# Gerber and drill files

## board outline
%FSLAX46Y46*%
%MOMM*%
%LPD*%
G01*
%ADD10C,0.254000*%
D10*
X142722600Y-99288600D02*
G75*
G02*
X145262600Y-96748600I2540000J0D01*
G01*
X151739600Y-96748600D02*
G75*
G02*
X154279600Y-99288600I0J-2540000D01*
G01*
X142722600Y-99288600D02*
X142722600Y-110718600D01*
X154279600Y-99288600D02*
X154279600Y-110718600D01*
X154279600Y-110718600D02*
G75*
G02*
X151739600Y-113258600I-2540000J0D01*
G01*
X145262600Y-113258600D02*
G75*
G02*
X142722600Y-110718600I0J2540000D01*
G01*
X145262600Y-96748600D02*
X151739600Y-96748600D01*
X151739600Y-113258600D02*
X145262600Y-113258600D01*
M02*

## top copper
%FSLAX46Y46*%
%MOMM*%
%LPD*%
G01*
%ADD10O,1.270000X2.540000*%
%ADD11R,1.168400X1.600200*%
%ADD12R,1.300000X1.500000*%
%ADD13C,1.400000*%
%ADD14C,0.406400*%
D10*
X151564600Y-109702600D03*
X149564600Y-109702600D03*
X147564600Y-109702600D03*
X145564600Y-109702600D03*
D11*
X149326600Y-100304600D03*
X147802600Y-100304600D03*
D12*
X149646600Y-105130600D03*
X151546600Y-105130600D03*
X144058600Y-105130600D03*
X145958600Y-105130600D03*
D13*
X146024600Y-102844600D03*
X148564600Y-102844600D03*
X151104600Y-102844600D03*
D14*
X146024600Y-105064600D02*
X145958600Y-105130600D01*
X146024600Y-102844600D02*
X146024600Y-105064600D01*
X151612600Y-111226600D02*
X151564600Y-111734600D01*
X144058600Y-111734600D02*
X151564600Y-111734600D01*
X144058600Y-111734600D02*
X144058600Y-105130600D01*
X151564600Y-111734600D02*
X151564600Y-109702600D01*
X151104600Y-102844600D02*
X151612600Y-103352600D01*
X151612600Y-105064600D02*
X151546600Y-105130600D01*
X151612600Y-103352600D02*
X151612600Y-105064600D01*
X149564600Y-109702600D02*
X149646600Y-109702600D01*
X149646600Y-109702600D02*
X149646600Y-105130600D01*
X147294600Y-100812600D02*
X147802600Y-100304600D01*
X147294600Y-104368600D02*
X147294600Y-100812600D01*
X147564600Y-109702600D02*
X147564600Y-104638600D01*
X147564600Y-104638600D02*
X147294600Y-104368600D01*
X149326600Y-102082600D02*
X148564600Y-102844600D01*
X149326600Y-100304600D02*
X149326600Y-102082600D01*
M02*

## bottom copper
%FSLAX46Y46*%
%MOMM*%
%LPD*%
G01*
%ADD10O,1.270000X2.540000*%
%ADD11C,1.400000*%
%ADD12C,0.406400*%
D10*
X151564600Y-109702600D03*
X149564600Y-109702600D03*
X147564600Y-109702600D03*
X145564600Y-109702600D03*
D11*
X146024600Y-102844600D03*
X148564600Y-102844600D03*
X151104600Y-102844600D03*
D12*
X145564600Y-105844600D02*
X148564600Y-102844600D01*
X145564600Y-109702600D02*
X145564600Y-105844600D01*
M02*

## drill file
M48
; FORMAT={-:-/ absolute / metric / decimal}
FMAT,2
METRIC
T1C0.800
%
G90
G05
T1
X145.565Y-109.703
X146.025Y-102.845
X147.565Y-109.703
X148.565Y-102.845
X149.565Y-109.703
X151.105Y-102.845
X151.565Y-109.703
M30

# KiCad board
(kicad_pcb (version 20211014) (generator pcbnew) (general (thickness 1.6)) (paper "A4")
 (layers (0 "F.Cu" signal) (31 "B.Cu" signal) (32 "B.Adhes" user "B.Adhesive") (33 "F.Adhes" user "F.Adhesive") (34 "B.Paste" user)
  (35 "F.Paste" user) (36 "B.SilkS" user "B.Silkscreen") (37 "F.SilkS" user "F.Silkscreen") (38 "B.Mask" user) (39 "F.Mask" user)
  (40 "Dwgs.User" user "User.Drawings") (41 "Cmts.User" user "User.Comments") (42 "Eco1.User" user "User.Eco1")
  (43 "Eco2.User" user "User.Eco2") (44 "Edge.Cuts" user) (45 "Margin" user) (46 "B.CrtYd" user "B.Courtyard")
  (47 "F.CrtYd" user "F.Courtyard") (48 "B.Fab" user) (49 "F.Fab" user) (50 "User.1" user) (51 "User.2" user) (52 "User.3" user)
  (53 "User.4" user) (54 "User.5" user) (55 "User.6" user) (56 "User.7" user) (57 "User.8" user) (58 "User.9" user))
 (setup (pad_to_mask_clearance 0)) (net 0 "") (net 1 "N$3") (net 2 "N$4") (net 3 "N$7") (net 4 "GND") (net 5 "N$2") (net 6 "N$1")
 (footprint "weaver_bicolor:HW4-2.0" (layer "F.Cu") (at 148.5646 109.7026 180)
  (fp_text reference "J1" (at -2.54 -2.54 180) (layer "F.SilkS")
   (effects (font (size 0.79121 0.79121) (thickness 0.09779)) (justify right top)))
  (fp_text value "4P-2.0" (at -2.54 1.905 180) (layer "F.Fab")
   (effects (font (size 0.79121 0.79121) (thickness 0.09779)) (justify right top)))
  (pad "1" thru_hole oval (at -3 0 270) (size 2.54 1.27) (drill 0.8) (layers *.Cu *.Mask) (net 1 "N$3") (solder_mask_margin 0.1016))
  (pad "2" thru_hole oval (at -1 0 270) (size 2.54 1.27) (drill 0.8) (layers *.Cu *.Mask) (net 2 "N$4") (solder_mask_margin 0.1016))
  (pad "3" thru_hole oval (at 1 0 270) (size 2.54 1.27) (drill 0.8) (layers *.Cu *.Mask) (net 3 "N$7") (solder_mask_margin 0.1016))
  (pad "4" thru_hole oval (at 3 0 270) (size 2.54 1.27) (drill 0.8) (layers *.Cu *.Mask) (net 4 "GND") (solder_mask_margin 0.1016)))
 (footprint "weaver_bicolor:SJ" (layer "F.Cu") (at 148.5646 100.3046 180)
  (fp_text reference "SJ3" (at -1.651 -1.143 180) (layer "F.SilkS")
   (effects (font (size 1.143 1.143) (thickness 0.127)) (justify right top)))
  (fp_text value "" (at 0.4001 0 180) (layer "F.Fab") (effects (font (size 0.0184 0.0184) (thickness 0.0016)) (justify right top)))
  (pad "1" smd rect (at -0.762 0 180) (size 1.1684 1.6002) (layers "F.Cu" "F.Paste" "F.Mask") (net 4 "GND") (solder_mask_margin 0.1016))
  (pad "2" smd rect (at 0.762 0 180) (size 1.1684 1.6002) (layers "F.Cu" "F.Paste" "F.Mask") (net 3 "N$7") (solder_mask_margin 0.1016)))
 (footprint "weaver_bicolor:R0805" (layer "F.Cu") (at 150.5966 105.1306)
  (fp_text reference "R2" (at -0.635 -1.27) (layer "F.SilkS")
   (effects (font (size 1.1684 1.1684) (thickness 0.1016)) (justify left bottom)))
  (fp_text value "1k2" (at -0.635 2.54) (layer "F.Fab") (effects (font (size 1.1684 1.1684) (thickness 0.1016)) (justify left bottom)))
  (pad "1" smd rect (at -0.95 0) (size 1.3 1.5) (layers "F.Cu" "F.Paste" "F.Mask") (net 2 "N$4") (solder_mask_margin 0.1016))
  (pad "2" smd rect (at 0.95 0) (size 1.3 1.5) (layers "F.Cu" "F.Paste" "F.Mask") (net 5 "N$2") (solder_mask_margin 0.1016)))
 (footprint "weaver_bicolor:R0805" (layer "F.Cu") (at 145.0086 105.1306)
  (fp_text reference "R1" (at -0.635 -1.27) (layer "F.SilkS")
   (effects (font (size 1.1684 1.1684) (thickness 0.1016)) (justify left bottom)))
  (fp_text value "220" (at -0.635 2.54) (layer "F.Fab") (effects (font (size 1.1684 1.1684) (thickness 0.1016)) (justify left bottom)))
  (pad "1" smd rect (at -0.95 0) (size 1.3 1.5) (layers "F.Cu" "F.Paste" "F.Mask") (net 1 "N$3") (solder_mask_margin 0.1016))
  (pad "2" smd rect (at 0.95 0) (size 1.3 1.5) (layers "F.Cu" "F.Paste" "F.Mask") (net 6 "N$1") (solder_mask_margin 0.1016)))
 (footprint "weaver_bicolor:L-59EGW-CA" (layer "B.Cu") (at 148.5646 102.8446 -90)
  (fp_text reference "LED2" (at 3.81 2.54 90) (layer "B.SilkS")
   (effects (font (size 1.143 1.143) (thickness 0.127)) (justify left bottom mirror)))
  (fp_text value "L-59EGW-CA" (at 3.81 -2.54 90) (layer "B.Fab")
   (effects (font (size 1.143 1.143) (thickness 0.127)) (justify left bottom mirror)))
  (pad "1" thru_hole circle (at 0 2.54 180) (size 1.4 1.4) (drill 0.8) (layers *.Cu *.Mask) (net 6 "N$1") (solder_mask_margin 0.1016))
  (pad "2" thru_hole circle (at 0 0 180) (size 1.4 1.4) (drill 0.8) (layers *.Cu *.Mask) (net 4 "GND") (solder_mask_margin 0.1016))
  (pad "3" thru_hole circle (at 0 -2.54 180) (size 1.4 1.4) (drill 0.8) (layers *.Cu *.Mask) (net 5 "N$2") (solder_mask_margin 0.1016)))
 (gr_arc (start 142.7226 99.2886) (mid 143.466549 97.492549) (end 145.2626 96.7486) (layer "Edge.Cuts") (width 0.254))
 (gr_arc (start 151.7396 96.7486) (mid 153.535651 97.492549) (end 154.2796 99.2886) (layer "Edge.Cuts") (width 0.254))
 (gr_line (start 142.7226 99.2886) (end 142.7226 110.7186) (layer "Edge.Cuts") (width 0.254))
 (gr_line (start 154.2796 99.2886) (end 154.2796 110.7186) (layer "Edge.Cuts") (width 0.254))
 (gr_arc (start 154.2796 110.7186) (mid 153.535651 112.514651) (end 151.7396 113.2586) (layer "Edge.Cuts") (width 0.254))
 (gr_arc (start 145.2626 113.2586) (mid 143.466549 112.514651) (end 142.7226 110.7186) (layer "Edge.Cuts") (width 0.254))
 (gr_line (start 145.2626 96.7486) (end 151.7396 96.7486) (layer "Edge.Cuts") (width 0.254))
 (gr_line (start 151.7396 113.2586) (end 145.2626 113.2586) (layer "Edge.Cuts") (width 0.254))
 (segment (start 146.0246 105.0646) (end 145.9586 105.1306) (width 0.4064) (layer "F.Cu") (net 6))
 (segment (start 146.0246 102.8446) (end 146.0246 105.0646) (width 0.4064) (layer "F.Cu") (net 6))
 (segment (start 151.6126 111.2266) (end 151.5646 111.7346) (width 0.4064) (layer "F.Cu") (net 1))
 (segment (start 144.0586 111.7346) (end 151.5646 111.7346) (width 0.4064) (layer "F.Cu") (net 1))
 (segment (start 144.0586 111.7346) (end 144.0586 105.1306) (width 0.4064) (layer "F.Cu") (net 1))
 (segment (start 151.5646 111.7346) (end 151.5646 109.7026) (width 0.4064) (layer "F.Cu") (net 1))
 (segment (start 151.1046 102.8446) (end 151.6126 103.3526) (width 0.4064) (layer "F.Cu") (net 5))
 (segment (start 151.6126 105.0646) (end 151.5466 105.1306) (width 0.4064) (layer "F.Cu") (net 5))
 (segment (start 151.6126 103.3526) (end 151.6126 105.0646) (width 0.4064) (layer "F.Cu") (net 5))
 (segment (start 149.5646 109.7026) (end 149.6466 109.7026) (width 0.4064) (layer "F.Cu") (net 2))
 (segment (start 149.6466 109.7026) (end 149.6466 105.1306) (width 0.4064) (layer "F.Cu") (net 2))
 (segment (start 147.2946 100.8126) (end 147.8026 100.3046) (width 0.4064) (layer "F.Cu") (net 3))
 (segment (start 147.2946 104.3686) (end 147.2946 100.8126) (width 0.4064) (layer "F.Cu") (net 3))
 (segment (start 147.5646 109.7026) (end 147.5646 104.6386) (width 0.4064) (layer "F.Cu") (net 3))
 (segment (start 147.5646 104.6386) (end 147.2946 104.3686) (width 0.4064) (layer "F.Cu") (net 3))
 (segment (start 149.3266 102.0826) (end 148.5646 102.8446) (width 0.4064) (layer "F.Cu") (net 4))
 (segment (start 149.3266 100.3046) (end 149.3266 102.0826) (width 0.4064) (layer "F.Cu") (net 4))
 (segment (start 145.5646 105.8446) (end 148.5646 102.8446) (width 0.4064) (layer "B.Cu") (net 4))
 (segment (start 145.5646 109.7026) (end 145.5646 105.8446) (width 0.4064) (layer "B.Cu") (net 4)))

